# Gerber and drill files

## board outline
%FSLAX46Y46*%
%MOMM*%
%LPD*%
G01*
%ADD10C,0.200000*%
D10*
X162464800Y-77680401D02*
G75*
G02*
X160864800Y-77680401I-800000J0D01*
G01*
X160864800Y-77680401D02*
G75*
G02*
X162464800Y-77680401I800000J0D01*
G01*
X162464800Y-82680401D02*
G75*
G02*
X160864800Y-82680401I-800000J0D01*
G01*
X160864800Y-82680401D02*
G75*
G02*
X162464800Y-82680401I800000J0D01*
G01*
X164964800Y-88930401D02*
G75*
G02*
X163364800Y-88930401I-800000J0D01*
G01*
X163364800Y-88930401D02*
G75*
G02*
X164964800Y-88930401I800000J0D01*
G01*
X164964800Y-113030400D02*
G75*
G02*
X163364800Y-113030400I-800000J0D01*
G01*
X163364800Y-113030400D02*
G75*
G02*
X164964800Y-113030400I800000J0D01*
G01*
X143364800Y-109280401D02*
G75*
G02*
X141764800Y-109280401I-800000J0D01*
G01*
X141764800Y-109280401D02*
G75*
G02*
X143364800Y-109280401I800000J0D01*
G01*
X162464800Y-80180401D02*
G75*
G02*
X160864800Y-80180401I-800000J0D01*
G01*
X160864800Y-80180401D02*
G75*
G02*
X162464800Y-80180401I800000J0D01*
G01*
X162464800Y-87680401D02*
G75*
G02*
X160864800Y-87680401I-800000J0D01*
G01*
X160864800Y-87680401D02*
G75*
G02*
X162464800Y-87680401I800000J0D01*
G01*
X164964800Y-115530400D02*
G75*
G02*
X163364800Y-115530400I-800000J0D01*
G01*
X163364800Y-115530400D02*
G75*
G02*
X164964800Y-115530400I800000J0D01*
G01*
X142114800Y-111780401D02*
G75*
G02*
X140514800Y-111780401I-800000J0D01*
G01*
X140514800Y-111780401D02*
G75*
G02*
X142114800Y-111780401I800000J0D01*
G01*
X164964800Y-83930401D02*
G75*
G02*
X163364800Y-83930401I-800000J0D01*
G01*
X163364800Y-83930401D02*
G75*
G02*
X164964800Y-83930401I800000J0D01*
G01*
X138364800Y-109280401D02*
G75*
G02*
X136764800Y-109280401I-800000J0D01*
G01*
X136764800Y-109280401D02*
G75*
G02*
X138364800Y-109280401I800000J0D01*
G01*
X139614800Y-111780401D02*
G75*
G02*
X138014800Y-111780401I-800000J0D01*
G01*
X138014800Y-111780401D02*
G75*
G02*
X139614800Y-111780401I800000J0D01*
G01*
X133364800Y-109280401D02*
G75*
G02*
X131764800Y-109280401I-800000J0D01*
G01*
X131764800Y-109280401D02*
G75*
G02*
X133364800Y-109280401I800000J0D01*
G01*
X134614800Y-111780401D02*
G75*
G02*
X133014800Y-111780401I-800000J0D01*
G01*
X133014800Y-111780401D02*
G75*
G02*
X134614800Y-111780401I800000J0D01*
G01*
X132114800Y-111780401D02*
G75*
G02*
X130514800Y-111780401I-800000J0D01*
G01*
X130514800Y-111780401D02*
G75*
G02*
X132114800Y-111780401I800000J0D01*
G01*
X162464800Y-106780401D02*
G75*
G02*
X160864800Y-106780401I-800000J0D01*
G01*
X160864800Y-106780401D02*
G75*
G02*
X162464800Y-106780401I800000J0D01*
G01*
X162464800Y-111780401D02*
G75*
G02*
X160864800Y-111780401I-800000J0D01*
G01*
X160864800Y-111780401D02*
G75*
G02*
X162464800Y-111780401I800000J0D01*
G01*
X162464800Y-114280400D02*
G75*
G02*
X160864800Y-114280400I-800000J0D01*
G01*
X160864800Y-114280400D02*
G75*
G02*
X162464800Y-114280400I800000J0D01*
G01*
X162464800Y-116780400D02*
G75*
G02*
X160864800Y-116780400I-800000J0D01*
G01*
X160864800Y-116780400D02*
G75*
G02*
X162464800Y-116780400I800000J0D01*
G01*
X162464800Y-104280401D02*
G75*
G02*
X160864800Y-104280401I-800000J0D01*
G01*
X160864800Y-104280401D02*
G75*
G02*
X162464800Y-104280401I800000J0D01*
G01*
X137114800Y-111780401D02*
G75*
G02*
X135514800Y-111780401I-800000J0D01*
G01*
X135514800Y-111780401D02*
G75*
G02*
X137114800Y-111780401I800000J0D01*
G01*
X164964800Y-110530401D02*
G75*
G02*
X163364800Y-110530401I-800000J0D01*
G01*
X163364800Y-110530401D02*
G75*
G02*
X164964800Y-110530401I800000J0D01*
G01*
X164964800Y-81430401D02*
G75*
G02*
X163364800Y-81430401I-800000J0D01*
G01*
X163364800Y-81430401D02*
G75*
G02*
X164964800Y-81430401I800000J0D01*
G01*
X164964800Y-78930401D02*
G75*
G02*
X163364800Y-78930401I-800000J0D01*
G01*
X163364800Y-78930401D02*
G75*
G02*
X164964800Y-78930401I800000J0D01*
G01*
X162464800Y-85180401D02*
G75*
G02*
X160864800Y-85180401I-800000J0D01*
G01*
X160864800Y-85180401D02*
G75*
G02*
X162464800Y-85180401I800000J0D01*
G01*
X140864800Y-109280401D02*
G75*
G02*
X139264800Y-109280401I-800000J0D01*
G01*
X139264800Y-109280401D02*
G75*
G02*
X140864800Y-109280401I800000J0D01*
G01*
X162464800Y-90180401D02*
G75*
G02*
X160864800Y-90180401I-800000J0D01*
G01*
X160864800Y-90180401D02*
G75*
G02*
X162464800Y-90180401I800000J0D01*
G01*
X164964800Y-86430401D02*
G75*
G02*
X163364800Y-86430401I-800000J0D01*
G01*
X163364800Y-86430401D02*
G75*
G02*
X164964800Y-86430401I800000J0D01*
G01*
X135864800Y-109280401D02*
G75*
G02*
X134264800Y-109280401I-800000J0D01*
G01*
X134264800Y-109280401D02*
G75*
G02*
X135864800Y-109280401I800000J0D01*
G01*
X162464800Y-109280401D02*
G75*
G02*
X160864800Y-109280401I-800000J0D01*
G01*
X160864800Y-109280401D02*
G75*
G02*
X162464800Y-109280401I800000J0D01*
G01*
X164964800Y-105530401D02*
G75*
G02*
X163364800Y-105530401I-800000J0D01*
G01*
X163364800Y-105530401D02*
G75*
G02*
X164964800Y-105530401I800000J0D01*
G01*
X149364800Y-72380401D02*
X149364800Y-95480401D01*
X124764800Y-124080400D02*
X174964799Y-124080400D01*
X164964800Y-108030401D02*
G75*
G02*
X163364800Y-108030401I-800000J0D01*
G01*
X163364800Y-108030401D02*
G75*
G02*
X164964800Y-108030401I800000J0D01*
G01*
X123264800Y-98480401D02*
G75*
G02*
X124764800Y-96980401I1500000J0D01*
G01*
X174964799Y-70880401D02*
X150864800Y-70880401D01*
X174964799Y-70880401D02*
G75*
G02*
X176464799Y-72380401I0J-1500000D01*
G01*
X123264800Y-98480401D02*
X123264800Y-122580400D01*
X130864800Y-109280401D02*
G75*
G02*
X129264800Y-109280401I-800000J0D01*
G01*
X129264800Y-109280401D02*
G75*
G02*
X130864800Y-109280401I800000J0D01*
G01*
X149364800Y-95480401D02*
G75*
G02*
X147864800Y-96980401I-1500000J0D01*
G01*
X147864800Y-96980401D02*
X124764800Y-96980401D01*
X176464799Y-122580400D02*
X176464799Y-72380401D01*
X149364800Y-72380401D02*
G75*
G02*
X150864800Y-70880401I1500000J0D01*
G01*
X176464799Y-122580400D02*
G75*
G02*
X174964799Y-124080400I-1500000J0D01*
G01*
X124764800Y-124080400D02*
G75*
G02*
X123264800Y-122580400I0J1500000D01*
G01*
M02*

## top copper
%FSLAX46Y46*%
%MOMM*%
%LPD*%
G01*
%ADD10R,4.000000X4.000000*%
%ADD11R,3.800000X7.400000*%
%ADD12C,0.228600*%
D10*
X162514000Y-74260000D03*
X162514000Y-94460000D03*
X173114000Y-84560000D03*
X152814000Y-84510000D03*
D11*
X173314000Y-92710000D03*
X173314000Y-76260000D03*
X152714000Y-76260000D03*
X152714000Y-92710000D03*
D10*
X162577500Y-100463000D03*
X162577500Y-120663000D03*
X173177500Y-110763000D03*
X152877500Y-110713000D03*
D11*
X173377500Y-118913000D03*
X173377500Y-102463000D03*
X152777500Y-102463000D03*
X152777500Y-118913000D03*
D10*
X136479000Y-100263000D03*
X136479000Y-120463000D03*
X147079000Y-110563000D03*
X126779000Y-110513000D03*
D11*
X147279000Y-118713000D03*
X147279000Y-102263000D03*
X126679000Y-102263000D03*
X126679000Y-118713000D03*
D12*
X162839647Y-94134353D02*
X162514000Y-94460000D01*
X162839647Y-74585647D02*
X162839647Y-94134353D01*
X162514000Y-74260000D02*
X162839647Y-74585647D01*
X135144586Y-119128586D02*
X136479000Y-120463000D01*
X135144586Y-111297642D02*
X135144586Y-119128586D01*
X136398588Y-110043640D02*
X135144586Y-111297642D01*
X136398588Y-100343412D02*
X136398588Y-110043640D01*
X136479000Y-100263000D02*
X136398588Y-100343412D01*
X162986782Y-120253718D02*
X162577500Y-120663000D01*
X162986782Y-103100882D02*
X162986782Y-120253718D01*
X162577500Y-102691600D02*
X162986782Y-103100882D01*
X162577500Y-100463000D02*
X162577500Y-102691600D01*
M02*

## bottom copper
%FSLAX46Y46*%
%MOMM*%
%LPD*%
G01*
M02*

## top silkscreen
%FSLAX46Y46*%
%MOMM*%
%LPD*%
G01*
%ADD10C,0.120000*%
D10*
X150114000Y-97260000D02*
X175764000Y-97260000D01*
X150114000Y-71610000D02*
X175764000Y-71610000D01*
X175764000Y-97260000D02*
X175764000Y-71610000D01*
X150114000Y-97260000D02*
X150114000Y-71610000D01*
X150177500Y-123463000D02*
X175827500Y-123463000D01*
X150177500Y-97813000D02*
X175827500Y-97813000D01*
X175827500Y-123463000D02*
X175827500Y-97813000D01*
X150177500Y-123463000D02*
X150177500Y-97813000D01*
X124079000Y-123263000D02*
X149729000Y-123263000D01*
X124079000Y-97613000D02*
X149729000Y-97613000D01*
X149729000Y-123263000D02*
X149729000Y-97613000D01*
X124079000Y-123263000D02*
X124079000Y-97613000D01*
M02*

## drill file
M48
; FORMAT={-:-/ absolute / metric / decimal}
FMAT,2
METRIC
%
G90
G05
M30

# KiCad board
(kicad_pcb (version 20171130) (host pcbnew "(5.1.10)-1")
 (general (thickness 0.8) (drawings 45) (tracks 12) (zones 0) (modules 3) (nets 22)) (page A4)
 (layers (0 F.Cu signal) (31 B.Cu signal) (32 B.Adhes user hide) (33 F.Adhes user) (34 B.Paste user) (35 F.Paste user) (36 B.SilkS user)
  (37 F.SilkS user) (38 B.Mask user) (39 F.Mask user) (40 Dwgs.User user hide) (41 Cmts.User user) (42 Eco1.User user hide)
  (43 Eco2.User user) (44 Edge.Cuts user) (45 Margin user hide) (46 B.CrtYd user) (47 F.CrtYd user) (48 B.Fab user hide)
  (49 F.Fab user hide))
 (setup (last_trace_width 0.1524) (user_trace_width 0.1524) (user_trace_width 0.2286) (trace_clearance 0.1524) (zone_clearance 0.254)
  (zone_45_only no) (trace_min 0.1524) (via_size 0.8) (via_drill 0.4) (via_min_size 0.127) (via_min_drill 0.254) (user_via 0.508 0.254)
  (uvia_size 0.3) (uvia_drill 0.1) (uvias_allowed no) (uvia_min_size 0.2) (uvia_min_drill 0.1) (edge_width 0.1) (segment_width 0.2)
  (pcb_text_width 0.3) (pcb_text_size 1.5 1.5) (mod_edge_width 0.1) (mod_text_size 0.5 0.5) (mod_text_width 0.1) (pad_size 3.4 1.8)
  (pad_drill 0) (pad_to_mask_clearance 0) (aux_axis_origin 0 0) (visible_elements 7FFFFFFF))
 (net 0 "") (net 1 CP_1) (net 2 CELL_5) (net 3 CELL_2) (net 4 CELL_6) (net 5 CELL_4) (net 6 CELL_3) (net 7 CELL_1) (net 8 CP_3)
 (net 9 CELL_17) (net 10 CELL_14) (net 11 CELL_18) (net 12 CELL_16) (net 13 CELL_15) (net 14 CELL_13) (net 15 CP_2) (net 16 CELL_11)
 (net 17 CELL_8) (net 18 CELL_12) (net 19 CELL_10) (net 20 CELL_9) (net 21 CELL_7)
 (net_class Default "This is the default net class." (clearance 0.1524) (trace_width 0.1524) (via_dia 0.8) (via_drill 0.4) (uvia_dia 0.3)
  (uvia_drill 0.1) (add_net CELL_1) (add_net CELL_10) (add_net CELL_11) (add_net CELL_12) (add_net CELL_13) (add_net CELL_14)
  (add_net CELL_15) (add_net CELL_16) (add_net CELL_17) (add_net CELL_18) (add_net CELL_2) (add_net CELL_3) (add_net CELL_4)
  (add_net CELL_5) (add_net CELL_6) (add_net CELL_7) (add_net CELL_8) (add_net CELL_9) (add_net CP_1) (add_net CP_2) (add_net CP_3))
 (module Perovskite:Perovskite (layer F.Cu) (at 150.114 97.26 90)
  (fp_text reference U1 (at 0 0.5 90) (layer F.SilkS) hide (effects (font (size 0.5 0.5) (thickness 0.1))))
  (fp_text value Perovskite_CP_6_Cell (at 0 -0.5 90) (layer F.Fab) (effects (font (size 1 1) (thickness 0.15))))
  (fp_line (start 0 0) (end 0 25.65) (layer F.SilkS) (width 0.12))
  (fp_line (start 25.65 0) (end 25.65 25.65) (layer F.SilkS) (width 0.12))
  (fp_line (start 0 25.65) (end 25.65 25.65) (layer F.SilkS) (width 0.12))
  (fp_line (start 0 0) (end 25.65 0) (layer F.SilkS) (width 0.12))
  (pad 7 smd rect (at 23 12.4 90) (size 4 4) (layers F.Cu F.Paste F.Mask) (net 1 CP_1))
  (pad 7 smd rect (at 2.8 12.4 90) (size 4 4) (layers F.Cu F.Paste F.Mask) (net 1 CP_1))
  (pad 5 smd rect (at 12.7 23 90) (size 4 4) (layers F.Cu F.Paste F.Mask) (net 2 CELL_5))
  (pad 2 smd rect (at 12.75 2.7 90) (size 4 4) (layers F.Cu F.Paste F.Mask) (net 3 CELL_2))
  (pad 6 smd rect (at 4.55 23.2 90) (size 7.4 3.8) (layers F.Cu F.Paste F.Mask) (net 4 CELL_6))
  (pad 4 smd rect (at 21 23.2 90) (size 7.4 3.8) (layers F.Cu F.Paste F.Mask) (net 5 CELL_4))
  (pad 3 smd rect (at 21 2.6 90) (size 7.4 3.8) (layers F.Cu F.Paste F.Mask) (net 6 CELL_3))
  (pad 1 smd rect (at 4.55 2.6 90) (size 7.4 3.8) (layers F.Cu F.Paste F.Mask) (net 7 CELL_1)))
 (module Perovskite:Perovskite (layer F.Cu) (at 150.1775 123.463 90)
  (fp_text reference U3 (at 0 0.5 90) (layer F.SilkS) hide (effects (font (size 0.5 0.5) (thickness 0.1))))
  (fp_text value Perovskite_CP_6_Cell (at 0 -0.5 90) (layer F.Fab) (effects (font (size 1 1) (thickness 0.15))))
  (fp_line (start 0 0) (end 0 25.65) (layer F.SilkS) (width 0.12))
  (fp_line (start 25.65 0) (end 25.65 25.65) (layer F.SilkS) (width 0.12))
  (fp_line (start 0 25.65) (end 25.65 25.65) (layer F.SilkS) (width 0.12))
  (fp_line (start 0 0) (end 25.65 0) (layer F.SilkS) (width 0.12))
  (pad 7 smd rect (at 23 12.4 90) (size 4 4) (layers F.Cu F.Paste F.Mask) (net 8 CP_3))
  (pad 7 smd rect (at 2.8 12.4 90) (size 4 4) (layers F.Cu F.Paste F.Mask) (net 8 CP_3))
  (pad 5 smd rect (at 12.7 23 90) (size 4 4) (layers F.Cu F.Paste F.Mask) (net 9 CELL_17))
  (pad 2 smd rect (at 12.75 2.7 90) (size 4 4) (layers F.Cu F.Paste F.Mask) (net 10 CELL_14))
  (pad 6 smd rect (at 4.55 23.2 90) (size 7.4 3.8) (layers F.Cu F.Paste F.Mask) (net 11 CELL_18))
  (pad 4 smd rect (at 21 23.2 90) (size 7.4 3.8) (layers F.Cu F.Paste F.Mask) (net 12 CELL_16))
  (pad 3 smd rect (at 21 2.6 90) (size 7.4 3.8) (layers F.Cu F.Paste F.Mask) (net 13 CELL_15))
  (pad 1 smd rect (at 4.55 2.6 90) (size 7.4 3.8) (layers F.Cu F.Paste F.Mask) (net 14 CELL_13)))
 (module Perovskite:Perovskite (layer F.Cu) (at 124.079 123.263 90)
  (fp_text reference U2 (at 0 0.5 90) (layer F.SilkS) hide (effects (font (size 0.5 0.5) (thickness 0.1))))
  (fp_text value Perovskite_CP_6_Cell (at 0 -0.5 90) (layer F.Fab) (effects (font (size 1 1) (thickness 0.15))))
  (fp_line (start 0 0) (end 0 25.65) (layer F.SilkS) (width 0.12))
  (fp_line (start 25.65 0) (end 25.65 25.65) (layer F.SilkS) (width 0.12))
  (fp_line (start 0 25.65) (end 25.65 25.65) (layer F.SilkS) (width 0.12))
  (fp_line (start 0 0) (end 25.65 0) (layer F.SilkS) (width 0.12))
  (pad 7 smd rect (at 23 12.4 90) (size 4 4) (layers F.Cu F.Paste F.Mask) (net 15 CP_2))
  (pad 7 smd rect (at 2.8 12.4 90) (size 4 4) (layers F.Cu F.Paste F.Mask) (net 15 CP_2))
  (pad 5 smd rect (at 12.7 23 90) (size 4 4) (layers F.Cu F.Paste F.Mask) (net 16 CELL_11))
  (pad 2 smd rect (at 12.75 2.7 90) (size 4 4) (layers F.Cu F.Paste F.Mask) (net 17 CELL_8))
  (pad 6 smd rect (at 4.55 23.2 90) (size 7.4 3.8) (layers F.Cu F.Paste F.Mask) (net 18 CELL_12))
  (pad 4 smd rect (at 21 23.2 90) (size 7.4 3.8) (layers F.Cu F.Paste F.Mask) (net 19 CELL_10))
  (pad 3 smd rect (at 21 2.6 90) (size 7.4 3.8) (layers F.Cu F.Paste F.Mask) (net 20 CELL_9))
  (pad 1 smd rect (at 4.55 2.6 90) (size 7.4 3.8) (layers F.Cu F.Paste F.Mask) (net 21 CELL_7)))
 (gr_circle (center 161.6648 77.680401) (end 162.4648 77.680401) (layer Edge.Cuts) (width 0.2))
 (gr_circle (center 161.6648 82.680401) (end 162.4648 82.680401) (layer Edge.Cuts) (width 0.2))
 (gr_circle (center 164.1648 88.930401) (end 164.9648 88.930401) (layer Edge.Cuts) (width 0.2))
 (gr_circle (center 164.1648 113.0304) (end 164.9648 113.0304) (layer Edge.Cuts) (width 0.2))
 (gr_circle (center 142.5648 109.280401) (end 143.3648 109.280401) (layer Edge.Cuts) (width 0.2))
 (gr_circle (center 161.6648 80.180401) (end 162.4648 80.180401) (layer Edge.Cuts) (width 0.2))
 (gr_circle (center 161.6648 87.680401) (end 162.4648 87.680401) (layer Edge.Cuts) (width 0.2))
 (gr_circle (center 164.1648 115.5304) (end 164.9648 115.5304) (layer Edge.Cuts) (width 0.2))
 (gr_circle (center 141.3148 111.780401) (end 142.1148 111.780401) (layer Edge.Cuts) (width 0.2))
 (gr_circle (center 164.1648 83.930401) (end 164.9648 83.930401) (layer Edge.Cuts) (width 0.2))
 (gr_circle (center 137.5648 109.280401) (end 138.3648 109.280401) (layer Edge.Cuts) (width 0.2))
 (gr_circle (center 138.8148 111.780401) (end 139.6148 111.780401) (layer Edge.Cuts) (width 0.2))
 (gr_circle (center 132.5648 109.280401) (end 133.3648 109.280401) (layer Edge.Cuts) (width 0.2))
 (gr_circle (center 133.8148 111.780401) (end 134.6148 111.780401) (layer Edge.Cuts) (width 0.2))
 (gr_circle (center 131.3148 111.780401) (end 132.1148 111.780401) (layer Edge.Cuts) (width 0.2))
 (gr_circle (center 161.6648 106.780401) (end 162.4648 106.780401) (layer Edge.Cuts) (width 0.2))
 (gr_circle (center 161.6648 111.780401) (end 162.4648 111.780401) (layer Edge.Cuts) (width 0.2))
 (gr_circle (center 161.6648 114.2804) (end 162.4648 114.2804) (layer Edge.Cuts) (width 0.2))
 (gr_circle (center 161.6648 116.7804) (end 162.4648 116.7804) (layer Edge.Cuts) (width 0.2))
 (gr_circle (center 161.6648 104.280401) (end 162.4648 104.280401) (layer Edge.Cuts) (width 0.2))
 (gr_circle (center 136.3148 111.780401) (end 137.1148 111.780401) (layer Edge.Cuts) (width 0.2))
 (gr_circle (center 164.1648 110.530401) (end 164.9648 110.530401) (layer Edge.Cuts) (width 0.2))
 (gr_circle (center 164.1648 81.430401) (end 164.9648 81.430401) (layer Edge.Cuts) (width 0.2))
 (gr_circle (center 164.1648 78.930401) (end 164.9648 78.930401) (layer Edge.Cuts) (width 0.2))
 (gr_circle (center 161.6648 85.180401) (end 162.4648 85.180401) (layer Edge.Cuts) (width 0.2))
 (gr_circle (center 140.0648 109.280401) (end 140.8648 109.280401) (layer Edge.Cuts) (width 0.2))
 (gr_circle (center 161.6648 90.180401) (end 162.4648 90.180401) (layer Edge.Cuts) (width 0.2))
 (gr_circle (center 164.1648 86.430401) (end 164.9648 86.430401) (layer Edge.Cuts) (width 0.2))
 (gr_circle (center 135.0648 109.280401) (end 135.8648 109.280401) (layer Edge.Cuts) (width 0.2))
 (gr_circle (center 161.6648 109.280401) (end 162.4648 109.280401) (layer Edge.Cuts) (width 0.2))
 (gr_circle (center 164.1648 105.530401) (end 164.9648 105.530401) (layer Edge.Cuts) (width 0.2))
 (gr_line (start 149.3648 72.380401) (end 149.3648 95.480401) (layer Edge.Cuts) (width 0.2))
 (gr_line (start 124.7648 124.0804) (end 174.964799 124.0804) (layer Edge.Cuts) (width 0.2))
 (gr_circle (center 164.1648 108.030401) (end 164.9648 108.030401) (layer Edge.Cuts) (width 0.2))
 (gr_arc (start 124.7648 98.480401) (end 124.7648 96.980401) (angle -90) (layer Edge.Cuts) (width 0.2))
 (gr_line (start 174.964799 70.880401) (end 150.8648 70.880401) (layer Edge.Cuts) (width 0.2))
 (gr_arc (start 174.964799 72.380401) (end 176.464799 72.380401) (angle -90) (layer Edge.Cuts) (width 0.2))
 (gr_line (start 123.2648 98.480401) (end 123.2648 122.5804) (layer Edge.Cuts) (width 0.2))
 (gr_circle (center 130.0648 109.280401) (end 130.8648 109.280401) (layer Edge.Cuts) (width 0.2))
 (gr_arc (start 147.8648 95.480401) (end 147.8648 96.980401) (angle -90) (layer Edge.Cuts) (width 0.2))
 (gr_line (start 147.8648 96.980401) (end 124.7648 96.980401) (layer Edge.Cuts) (width 0.2))
 (gr_line (start 176.464799 122.5804) (end 176.464799 72.380401) (layer Edge.Cuts) (width 0.2))
 (gr_arc (start 150.8648 72.380401) (end 150.8648 70.880401) (angle -90) (layer Edge.Cuts) (width 0.2))
 (gr_arc (start 174.964799 122.5804) (end 174.964799 124.0804) (angle -90) (layer Edge.Cuts) (width 0.2))
 (gr_arc (start 124.7648 122.5804) (end 123.2648 122.5804) (angle -90) (layer Edge.Cuts) (width 0.2))
 (segment (start 162.839647 94.134353) (end 162.514 94.46) (width 0.2286) (layer F.Cu) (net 1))
 (segment (start 162.839647 74.585647) (end 162.839647 94.134353) (width 0.2286) (layer F.Cu) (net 1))
 (segment (start 162.514 74.26) (end 162.839647 74.585647) (width 0.2286) (layer F.Cu) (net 1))
 (segment (start 135.144586 119.128586) (end 136.479 120.463) (width 0.2286) (layer F.Cu) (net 15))
 (segment (start 135.144586 111.297642) (end 135.144586 119.128586) (width 0.2286) (layer F.Cu) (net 15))
 (segment (start 136.398588 110.04364) (end 135.144586 111.297642) (width 0.2286) (layer F.Cu) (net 15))
 (segment (start 136.398588 100.343412) (end 136.398588 110.04364) (width 0.2286) (layer F.Cu) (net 15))
 (segment (start 136.479 100.263) (end 136.398588 100.343412) (width 0.2286) (layer F.Cu) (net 15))
 (segment (start 162.986782 120.253718) (end 162.5775 120.663) (width 0.2286) (layer F.Cu) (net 8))
 (segment (start 162.986782 103.100882) (end 162.986782 120.253718) (width 0.2286) (layer F.Cu) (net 8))
 (segment (start 162.5775 102.6916) (end 162.986782 103.100882) (width 0.2286) (layer F.Cu) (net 8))
 (segment (start 162.5775 100.463) (end 162.5775 102.6916) (width 0.2286) (layer F.Cu) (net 8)))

